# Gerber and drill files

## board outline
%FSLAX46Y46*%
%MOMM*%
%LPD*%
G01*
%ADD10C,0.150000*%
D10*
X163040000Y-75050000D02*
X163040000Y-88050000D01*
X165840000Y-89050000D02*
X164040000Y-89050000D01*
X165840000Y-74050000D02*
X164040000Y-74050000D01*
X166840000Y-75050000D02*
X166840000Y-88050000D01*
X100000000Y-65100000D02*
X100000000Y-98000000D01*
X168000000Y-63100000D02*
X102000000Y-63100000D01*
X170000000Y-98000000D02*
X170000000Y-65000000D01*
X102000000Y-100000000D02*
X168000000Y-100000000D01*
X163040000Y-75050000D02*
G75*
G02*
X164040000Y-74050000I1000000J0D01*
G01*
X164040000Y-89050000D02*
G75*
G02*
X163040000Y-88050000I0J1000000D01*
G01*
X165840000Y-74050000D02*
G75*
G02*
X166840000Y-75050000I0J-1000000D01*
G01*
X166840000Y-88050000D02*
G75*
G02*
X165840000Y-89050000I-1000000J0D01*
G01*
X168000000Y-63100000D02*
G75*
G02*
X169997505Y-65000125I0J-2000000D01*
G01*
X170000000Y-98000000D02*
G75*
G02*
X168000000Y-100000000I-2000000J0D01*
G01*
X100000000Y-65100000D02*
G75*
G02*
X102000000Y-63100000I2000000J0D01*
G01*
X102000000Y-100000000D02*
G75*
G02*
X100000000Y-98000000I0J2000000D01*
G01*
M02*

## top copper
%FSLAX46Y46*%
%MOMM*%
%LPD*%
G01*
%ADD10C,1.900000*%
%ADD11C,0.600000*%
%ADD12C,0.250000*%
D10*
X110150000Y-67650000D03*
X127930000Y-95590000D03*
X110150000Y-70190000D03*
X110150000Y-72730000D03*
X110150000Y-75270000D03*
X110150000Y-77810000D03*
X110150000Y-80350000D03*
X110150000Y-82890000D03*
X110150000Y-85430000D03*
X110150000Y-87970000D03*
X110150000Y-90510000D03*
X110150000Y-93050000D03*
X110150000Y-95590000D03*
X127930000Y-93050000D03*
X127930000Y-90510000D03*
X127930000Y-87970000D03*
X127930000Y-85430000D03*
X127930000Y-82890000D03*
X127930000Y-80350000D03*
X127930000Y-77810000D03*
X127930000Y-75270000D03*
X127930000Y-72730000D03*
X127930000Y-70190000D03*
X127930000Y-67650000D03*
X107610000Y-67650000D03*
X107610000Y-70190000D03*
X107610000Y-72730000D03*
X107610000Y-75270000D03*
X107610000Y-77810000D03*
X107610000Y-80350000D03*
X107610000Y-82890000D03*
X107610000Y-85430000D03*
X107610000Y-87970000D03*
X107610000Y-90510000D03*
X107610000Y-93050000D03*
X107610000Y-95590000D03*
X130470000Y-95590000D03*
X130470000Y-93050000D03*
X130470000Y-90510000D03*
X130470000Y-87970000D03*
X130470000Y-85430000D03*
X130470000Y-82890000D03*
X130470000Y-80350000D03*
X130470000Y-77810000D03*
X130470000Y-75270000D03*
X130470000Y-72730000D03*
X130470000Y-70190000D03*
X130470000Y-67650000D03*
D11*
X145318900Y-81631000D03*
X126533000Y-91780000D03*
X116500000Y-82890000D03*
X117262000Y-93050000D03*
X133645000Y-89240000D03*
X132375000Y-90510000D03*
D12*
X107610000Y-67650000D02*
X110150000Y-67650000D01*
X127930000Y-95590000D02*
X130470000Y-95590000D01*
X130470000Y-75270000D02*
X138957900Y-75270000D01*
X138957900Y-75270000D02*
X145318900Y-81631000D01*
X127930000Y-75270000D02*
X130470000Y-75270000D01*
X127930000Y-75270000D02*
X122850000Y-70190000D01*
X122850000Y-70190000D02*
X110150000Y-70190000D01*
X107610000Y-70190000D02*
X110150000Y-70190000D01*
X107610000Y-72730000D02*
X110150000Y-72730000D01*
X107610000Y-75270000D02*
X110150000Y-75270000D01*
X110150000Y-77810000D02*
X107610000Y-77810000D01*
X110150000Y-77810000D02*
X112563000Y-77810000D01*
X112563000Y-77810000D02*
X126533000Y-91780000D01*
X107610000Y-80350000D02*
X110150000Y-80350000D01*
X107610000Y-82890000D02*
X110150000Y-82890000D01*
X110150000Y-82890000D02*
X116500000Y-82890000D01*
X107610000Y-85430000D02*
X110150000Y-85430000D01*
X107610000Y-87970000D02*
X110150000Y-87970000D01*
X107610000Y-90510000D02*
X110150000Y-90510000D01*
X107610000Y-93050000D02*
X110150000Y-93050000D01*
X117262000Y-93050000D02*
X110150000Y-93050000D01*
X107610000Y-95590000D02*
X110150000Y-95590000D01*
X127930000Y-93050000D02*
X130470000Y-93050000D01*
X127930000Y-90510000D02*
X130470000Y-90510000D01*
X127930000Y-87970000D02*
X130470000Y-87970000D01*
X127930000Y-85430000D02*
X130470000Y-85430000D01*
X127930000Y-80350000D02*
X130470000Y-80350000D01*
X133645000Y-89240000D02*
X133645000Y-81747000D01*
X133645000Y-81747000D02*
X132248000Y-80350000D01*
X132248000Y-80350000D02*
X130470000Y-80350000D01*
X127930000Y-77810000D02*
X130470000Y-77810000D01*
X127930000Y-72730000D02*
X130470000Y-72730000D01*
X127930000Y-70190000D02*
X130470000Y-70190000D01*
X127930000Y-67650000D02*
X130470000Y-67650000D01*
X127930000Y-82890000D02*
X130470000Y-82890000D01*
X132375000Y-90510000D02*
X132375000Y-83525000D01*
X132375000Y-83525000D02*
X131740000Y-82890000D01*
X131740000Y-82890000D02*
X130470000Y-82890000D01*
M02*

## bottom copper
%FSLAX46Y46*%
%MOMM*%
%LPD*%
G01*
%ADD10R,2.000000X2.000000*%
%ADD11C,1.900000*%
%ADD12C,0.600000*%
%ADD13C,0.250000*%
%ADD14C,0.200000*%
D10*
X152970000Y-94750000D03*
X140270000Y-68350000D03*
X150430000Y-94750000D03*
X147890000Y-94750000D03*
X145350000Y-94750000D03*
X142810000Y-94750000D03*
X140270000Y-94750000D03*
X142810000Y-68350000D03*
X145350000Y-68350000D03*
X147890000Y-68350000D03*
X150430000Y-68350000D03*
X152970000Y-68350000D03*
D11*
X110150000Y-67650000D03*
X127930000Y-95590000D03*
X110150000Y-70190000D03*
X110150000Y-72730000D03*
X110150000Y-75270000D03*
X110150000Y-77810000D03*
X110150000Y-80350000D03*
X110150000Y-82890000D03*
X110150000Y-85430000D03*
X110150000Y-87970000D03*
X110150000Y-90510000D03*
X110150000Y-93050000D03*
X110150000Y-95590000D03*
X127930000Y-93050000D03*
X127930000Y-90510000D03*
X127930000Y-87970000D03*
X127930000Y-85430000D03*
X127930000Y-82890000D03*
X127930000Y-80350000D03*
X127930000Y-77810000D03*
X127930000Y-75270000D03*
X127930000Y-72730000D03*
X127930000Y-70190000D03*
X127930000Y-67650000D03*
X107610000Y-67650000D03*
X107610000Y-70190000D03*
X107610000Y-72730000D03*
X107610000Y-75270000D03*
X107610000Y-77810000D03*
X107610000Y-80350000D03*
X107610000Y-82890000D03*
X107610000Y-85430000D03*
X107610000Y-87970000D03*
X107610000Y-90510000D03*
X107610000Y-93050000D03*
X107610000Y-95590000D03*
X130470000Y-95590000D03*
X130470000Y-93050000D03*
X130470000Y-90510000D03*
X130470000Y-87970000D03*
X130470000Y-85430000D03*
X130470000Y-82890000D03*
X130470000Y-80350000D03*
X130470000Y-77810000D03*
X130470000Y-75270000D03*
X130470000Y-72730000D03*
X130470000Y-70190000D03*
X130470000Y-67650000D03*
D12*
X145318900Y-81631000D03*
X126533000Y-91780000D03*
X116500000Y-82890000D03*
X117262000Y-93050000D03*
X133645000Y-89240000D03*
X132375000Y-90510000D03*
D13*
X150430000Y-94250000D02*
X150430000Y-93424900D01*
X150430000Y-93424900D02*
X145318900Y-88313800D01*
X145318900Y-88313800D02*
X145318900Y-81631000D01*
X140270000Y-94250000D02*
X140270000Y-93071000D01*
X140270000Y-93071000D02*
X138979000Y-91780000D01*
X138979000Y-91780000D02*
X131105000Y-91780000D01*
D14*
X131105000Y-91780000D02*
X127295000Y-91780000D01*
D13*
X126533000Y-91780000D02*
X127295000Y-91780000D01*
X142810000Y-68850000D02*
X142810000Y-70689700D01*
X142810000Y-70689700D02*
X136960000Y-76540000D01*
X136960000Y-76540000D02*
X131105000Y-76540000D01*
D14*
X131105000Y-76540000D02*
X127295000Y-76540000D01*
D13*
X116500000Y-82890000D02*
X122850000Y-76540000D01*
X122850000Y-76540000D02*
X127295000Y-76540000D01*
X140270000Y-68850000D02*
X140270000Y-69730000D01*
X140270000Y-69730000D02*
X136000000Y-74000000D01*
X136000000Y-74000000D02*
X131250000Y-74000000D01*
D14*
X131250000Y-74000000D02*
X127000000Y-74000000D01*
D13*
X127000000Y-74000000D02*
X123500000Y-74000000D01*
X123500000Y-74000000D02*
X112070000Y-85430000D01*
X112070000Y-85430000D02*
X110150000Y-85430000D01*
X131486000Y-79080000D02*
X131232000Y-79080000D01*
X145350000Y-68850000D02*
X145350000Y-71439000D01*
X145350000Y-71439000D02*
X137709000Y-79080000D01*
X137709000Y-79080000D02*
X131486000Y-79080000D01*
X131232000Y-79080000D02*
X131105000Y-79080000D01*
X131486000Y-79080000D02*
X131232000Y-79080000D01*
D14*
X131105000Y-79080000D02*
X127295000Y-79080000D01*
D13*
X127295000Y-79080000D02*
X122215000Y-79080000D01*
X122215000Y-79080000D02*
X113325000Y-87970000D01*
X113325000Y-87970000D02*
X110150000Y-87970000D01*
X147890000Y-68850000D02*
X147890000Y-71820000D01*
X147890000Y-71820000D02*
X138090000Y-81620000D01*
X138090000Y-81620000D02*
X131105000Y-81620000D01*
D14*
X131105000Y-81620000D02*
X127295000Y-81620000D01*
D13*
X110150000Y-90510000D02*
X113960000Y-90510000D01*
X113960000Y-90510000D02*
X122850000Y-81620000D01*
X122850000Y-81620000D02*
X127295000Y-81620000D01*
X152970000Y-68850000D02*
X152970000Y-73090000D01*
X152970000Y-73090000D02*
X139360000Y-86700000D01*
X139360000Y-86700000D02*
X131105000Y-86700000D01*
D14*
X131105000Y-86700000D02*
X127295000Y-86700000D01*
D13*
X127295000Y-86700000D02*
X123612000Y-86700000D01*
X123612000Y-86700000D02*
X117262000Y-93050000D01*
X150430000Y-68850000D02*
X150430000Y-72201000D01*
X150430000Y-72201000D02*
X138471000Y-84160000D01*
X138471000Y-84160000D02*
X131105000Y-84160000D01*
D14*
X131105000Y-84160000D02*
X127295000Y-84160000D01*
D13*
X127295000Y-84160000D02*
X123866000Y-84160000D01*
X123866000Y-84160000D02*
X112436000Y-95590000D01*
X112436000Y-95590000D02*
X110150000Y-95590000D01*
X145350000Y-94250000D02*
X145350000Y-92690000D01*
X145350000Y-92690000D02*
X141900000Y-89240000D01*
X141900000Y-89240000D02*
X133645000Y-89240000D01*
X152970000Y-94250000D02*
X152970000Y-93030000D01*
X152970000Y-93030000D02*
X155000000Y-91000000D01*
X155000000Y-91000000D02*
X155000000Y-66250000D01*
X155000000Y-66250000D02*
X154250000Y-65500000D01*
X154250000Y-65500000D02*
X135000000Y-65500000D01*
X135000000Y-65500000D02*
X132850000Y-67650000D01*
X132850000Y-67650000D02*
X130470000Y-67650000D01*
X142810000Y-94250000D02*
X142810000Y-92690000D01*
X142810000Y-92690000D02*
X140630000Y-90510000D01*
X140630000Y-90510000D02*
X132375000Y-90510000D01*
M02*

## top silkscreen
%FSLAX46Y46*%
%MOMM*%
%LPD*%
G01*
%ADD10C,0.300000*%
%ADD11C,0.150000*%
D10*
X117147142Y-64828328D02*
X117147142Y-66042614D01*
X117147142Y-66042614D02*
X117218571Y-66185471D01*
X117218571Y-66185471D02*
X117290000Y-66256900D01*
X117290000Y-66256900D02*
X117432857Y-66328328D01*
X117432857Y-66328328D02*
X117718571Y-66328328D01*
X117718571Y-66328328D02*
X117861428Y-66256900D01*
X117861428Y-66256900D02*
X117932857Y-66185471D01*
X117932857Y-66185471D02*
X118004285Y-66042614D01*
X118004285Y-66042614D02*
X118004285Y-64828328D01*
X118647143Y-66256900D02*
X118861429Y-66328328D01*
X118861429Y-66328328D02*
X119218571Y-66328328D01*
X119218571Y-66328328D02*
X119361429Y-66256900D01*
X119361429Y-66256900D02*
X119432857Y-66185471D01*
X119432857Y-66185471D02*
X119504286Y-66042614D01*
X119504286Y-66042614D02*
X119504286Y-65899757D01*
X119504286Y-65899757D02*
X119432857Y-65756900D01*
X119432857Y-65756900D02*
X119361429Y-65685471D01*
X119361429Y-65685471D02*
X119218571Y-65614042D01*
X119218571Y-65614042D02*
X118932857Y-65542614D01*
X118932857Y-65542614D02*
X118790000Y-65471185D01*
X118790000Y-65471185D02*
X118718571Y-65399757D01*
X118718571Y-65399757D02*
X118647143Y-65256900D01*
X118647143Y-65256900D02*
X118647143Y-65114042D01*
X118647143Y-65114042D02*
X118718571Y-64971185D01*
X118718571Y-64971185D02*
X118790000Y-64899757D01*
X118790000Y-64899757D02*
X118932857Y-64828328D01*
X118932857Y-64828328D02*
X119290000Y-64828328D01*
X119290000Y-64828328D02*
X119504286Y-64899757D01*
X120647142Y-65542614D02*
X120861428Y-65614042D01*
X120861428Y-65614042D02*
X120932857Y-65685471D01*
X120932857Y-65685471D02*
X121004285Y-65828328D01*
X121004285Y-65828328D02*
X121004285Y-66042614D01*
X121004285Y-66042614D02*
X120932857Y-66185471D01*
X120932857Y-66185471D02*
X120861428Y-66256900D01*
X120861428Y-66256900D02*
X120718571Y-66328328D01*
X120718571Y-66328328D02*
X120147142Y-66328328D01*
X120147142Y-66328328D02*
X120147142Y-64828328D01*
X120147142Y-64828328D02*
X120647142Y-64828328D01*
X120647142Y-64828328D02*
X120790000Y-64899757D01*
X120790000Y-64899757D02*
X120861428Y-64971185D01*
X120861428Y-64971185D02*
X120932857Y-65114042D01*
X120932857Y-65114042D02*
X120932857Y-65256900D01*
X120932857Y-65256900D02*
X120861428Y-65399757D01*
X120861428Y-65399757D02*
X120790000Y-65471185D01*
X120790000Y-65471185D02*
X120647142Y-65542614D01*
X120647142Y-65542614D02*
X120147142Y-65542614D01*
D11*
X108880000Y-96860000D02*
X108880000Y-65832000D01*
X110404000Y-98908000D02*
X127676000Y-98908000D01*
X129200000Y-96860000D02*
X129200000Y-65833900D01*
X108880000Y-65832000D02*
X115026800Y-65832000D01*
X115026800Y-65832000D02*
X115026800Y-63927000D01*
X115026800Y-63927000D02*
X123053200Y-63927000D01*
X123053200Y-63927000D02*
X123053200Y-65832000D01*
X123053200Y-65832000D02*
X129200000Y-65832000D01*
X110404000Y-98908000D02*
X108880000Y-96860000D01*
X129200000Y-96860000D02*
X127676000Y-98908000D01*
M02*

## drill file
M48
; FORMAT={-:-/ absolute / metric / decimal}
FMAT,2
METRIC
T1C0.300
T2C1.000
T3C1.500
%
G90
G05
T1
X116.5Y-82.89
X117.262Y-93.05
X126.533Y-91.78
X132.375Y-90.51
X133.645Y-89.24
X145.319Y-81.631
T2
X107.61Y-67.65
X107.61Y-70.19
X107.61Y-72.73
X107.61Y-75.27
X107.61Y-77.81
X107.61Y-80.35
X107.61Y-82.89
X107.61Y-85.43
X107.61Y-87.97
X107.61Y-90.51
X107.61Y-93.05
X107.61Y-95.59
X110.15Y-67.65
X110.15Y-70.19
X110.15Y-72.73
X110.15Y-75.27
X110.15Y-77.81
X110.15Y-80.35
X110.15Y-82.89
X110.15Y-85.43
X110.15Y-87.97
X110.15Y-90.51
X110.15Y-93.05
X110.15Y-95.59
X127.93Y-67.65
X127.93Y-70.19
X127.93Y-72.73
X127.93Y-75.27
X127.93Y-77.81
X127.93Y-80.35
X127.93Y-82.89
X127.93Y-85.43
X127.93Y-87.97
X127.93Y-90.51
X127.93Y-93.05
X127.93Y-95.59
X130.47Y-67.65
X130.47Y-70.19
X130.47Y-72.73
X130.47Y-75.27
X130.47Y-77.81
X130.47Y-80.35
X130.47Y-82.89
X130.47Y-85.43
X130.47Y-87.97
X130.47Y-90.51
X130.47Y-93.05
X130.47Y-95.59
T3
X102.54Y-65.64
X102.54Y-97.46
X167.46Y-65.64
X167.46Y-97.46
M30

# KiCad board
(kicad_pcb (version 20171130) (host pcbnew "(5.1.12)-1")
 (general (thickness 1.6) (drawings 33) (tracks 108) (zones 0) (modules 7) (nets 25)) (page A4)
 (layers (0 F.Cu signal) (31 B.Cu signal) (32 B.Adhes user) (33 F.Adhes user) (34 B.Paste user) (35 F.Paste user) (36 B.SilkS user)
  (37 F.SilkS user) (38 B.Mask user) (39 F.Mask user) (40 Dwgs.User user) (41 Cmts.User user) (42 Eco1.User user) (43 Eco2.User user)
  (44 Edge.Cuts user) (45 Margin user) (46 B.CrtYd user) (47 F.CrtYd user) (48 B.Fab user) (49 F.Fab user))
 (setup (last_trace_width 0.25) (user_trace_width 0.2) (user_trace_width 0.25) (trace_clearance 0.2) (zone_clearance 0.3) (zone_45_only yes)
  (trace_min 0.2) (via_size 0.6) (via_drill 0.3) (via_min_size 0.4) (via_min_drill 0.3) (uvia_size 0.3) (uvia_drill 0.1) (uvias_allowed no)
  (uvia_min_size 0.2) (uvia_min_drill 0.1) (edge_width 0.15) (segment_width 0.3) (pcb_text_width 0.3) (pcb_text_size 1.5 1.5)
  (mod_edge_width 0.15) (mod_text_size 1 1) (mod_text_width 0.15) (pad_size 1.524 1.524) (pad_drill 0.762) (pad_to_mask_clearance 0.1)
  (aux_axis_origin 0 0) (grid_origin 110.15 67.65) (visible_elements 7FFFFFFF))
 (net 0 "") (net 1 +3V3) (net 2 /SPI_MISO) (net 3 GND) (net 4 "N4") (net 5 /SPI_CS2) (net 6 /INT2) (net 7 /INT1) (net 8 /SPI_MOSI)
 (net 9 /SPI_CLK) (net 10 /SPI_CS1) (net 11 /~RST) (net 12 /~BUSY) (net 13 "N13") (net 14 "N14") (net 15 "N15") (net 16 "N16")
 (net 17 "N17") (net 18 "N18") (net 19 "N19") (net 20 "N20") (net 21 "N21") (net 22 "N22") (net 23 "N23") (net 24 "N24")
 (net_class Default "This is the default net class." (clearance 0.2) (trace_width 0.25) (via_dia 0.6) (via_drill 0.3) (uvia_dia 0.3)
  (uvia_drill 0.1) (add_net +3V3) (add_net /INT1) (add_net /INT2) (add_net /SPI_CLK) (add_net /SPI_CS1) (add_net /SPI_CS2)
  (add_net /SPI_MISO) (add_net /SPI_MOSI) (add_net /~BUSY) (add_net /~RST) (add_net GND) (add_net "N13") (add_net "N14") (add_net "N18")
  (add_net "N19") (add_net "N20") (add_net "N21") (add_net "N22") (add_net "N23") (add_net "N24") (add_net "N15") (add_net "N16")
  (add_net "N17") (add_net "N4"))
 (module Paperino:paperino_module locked (layer B.Cu) (at 149.57 81.55 90)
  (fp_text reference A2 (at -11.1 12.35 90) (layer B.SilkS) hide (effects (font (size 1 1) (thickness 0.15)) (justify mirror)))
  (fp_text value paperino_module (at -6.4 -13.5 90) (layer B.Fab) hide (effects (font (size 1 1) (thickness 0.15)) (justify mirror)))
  (pad 1 smd rect (at -12.7 3.4 90) (size 2 2) (drill (offset -0.5 0)) (layers B.Cu B.Paste B.Mask) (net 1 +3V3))
  (pad 7 smd rect (at 12.7 -9.3 90) (size 2 2) (drill (offset 0.5 0)) (layers B.Cu B.Paste B.Mask) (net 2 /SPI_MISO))
  (pad 2 smd rect (at -12.7 0.86 90) (size 2 2) (drill (offset -0.5 0)) (layers B.Cu B.Paste B.Mask) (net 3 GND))
  (pad 3 smd rect (at -12.7 -1.68 90) (size 2 2) (drill (offset -0.5 0)) (layers B.Cu B.Paste B.Mask) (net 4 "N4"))
  (pad 4 smd rect (at -12.7 -4.22 90) (size 2 2) (drill (offset -0.5 0)) (layers B.Cu B.Paste B.Mask) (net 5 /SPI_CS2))
  (pad 5 smd rect (at -12.7 -6.76 90) (size 2 2) (drill (offset -0.5 0)) (layers B.Cu B.Paste B.Mask) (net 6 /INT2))
  (pad 6 smd rect (at -12.7 -9.3 90) (size 2 2) (drill (offset -0.5 0)) (layers B.Cu B.Paste B.Mask) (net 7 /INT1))
  (pad 8 smd rect (at 12.7 -6.76 90) (size 2 2) (drill (offset 0.5 0)) (layers B.Cu B.Paste B.Mask) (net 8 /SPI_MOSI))
  (pad 9 smd rect (at 12.7 -4.22 90) (size 2 2) (drill (offset 0.5 0)) (layers B.Cu B.Paste B.Mask) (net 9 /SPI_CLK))
  (pad 10 smd rect (at 12.7 -1.68 90) (size 2 2) (drill (offset 0.5 0)) (layers B.Cu B.Paste B.Mask) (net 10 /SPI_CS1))
  (pad 11 smd rect (at 12.7 0.86 90) (size 2 2) (drill (offset 0.5 0)) (layers B.Cu B.Paste B.Mask) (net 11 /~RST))
  (pad 12 smd rect (at 12.7 3.4 90) (size 2 2) (drill (offset 0.5 0)) (layers B.Cu B.Paste B.Mask) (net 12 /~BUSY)))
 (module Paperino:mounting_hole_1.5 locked (layer F.Cu) (at 102.54 97.46)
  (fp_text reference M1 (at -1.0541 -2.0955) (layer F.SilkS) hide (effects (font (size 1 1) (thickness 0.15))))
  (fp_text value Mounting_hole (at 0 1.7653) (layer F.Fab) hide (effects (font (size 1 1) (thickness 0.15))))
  (pad "" np_thru_hole circle (at 0 0) (size 1.5 1.5) (drill 1.5) (layers *.Cu *.Mask)))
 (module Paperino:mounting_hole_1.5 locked (layer F.Cu) (at 167.46 65.64)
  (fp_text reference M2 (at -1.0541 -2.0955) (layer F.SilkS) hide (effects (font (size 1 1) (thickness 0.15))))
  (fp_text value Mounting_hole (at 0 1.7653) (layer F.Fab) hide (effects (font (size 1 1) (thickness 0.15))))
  (pad "" np_thru_hole circle (at 0 0) (size 1.5 1.5) (drill 1.5) (layers *.Cu *.Mask)))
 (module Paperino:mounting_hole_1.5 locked (layer F.Cu) (at 102.54 65.64)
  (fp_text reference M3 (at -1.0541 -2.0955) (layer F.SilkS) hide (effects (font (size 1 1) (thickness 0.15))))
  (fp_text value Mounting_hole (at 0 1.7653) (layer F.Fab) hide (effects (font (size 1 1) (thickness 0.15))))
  (pad "" np_thru_hole circle (at 0 0) (size 1.5 1.5) (drill 1.5) (layers *.Cu *.Mask)))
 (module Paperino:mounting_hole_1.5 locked (layer F.Cu) (at 167.46 97.46)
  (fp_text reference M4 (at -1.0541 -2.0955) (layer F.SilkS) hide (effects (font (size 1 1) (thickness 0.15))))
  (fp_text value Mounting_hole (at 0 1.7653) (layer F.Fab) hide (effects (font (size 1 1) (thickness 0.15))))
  (pad "" np_thru_hole circle (at 0 0) (size 1.5 1.5) (drill 1.5) (layers *.Cu *.Mask)))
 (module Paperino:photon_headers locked (layer F.Cu) (at 108.88 99.908)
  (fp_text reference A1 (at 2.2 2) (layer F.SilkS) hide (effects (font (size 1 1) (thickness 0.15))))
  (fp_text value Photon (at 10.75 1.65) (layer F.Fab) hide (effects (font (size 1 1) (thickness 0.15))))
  (fp_line (start 0 -3.048) (end 0 -34.076) (layer F.SilkS) (width 0.15))
  (fp_line (start 1.524 -1) (end 18.796 -1) (layer F.SilkS) (width 0.15))
  (fp_line (start 20.32 -3.048) (end 20.32 -34.0741) (layer F.SilkS) (width 0.15))
  (fp_line (start 0 -34.076) (end 6.1468 -34.076) (layer F.SilkS) (width 0.15))
  (fp_line (start 6.1468 -34.076) (end 6.1468 -35.981) (layer F.SilkS) (width 0.15))
  (fp_line (start 6.1468 -35.981) (end 14.1732 -35.981) (layer F.SilkS) (width 0.15))
  (fp_line (start 14.1732 -35.981) (end 14.1732 -34.076) (layer F.SilkS) (width 0.15))
  (fp_line (start 14.1732 -34.076) (end 20.32 -34.076) (layer F.SilkS) (width 0.15))
  (fp_line (start 1.524 -1) (end 0 -3.048) (layer F.SilkS) (width 0.15))
  (fp_line (start 20.32 -3.048) (end 18.796 -1) (layer F.SilkS) (width 0.15))
  (pad 1 thru_hole circle (at 1.27 -32.258) (size 1.9 1.9) (drill 1) (layers *.Cu *.Mask) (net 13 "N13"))
  (pad 13 thru_hole circle (at 19.05 -4.318) (size 1.9 1.9) (drill 1) (layers *.Cu *.Mask) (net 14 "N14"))
  (pad 2 thru_hole circle (at 1.27 -29.718) (size 1.9 1.9) (drill 1) (layers *.Cu *.Mask) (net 3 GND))
  (pad 3 thru_hole circle (at 1.27 -27.178) (size 1.9 1.9) (drill 1) (layers *.Cu *.Mask) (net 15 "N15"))
  (pad 4 thru_hole circle (at 1.27 -24.638) (size 1.9 1.9) (drill 1) (layers *.Cu *.Mask) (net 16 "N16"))
  (pad 5 thru_hole circle (at 1.27 -22.098) (size 1.9 1.9) (drill 1) (layers *.Cu *.Mask) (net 7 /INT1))
  (pad 6 thru_hole circle (at 1.27 -19.558) (size 1.9 1.9) (drill 1) (layers *.Cu *.Mask) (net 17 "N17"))
  (pad 7 thru_hole circle (at 1.27 -17.018) (size 1.9 1.9) (drill 1) (layers *.Cu *.Mask) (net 8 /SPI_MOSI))
  (pad 8 thru_hole circle (at 1.27 -14.478) (size 1.9 1.9) (drill 1) (layers *.Cu *.Mask) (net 2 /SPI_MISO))
  (pad 9 thru_hole circle (at 1.27 -11.938) (size 1.9 1.9) (drill 1) (layers *.Cu *.Mask) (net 9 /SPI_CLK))
  (pad 10 thru_hole circle (at 1.27 -9.398) (size 1.9 1.9) (drill 1) (layers *.Cu *.Mask) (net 10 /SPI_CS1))
  (pad 11 thru_hole circle (at 1.27 -6.858) (size 1.9 1.9) (drill 1) (layers *.Cu *.Mask) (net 12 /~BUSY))
  (pad 12 thru_hole circle (at 1.27 -4.318) (size 1.9 1.9) (drill 1) (layers *.Cu *.Mask) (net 11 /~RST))
  (pad 14 thru_hole circle (at 19.05 -6.858) (size 1.9 1.9) (drill 1) (layers *.Cu *.Mask) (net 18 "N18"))
  (pad 15 thru_hole circle (at 19.05 -9.398) (size 1.9 1.9) (drill 1) (layers *.Cu *.Mask) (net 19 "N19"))
  (pad 16 thru_hole circle (at 19.05 -11.938) (size 1.9 1.9) (drill 1) (layers *.Cu *.Mask) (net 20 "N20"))
  (pad 17 thru_hole circle (at 19.05 -14.478) (size 1.9 1.9) (drill 1) (layers *.Cu *.Mask) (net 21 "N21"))
  (pad 18 thru_hole circle (at 19.05 -17.018) (size 1.9 1.9) (drill 1) (layers *.Cu *.Mask) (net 6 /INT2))
  (pad 19 thru_hole circle (at 19.05 -19.558) (size 1.9 1.9) (drill 1) (layers *.Cu *.Mask) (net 5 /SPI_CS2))
  (pad 20 thru_hole circle (at 19.05 -22.098) (size 1.9 1.9) (drill 1) (layers *.Cu *.Mask) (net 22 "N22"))
  (pad 21 thru_hole circle (at 19.05 -24.638) (size 1.9 1.9) (drill 1) (layers *.Cu *.Mask) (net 3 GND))
  (pad 22 thru_hole circle (at 19.05 -27.178) (size 1.9 1.9) (drill 1) (layers *.Cu *.Mask) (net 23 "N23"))
  (pad 23 thru_hole circle (at 19.05 -29.718) (size 1.9 1.9) (drill 1) (layers *.Cu *.Mask) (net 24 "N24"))
  (pad 24 thru_hole circle (at 19.05 -32.258) (size 1.9 1.9) (drill 1) (layers *.Cu *.Mask) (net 1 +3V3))
  (pad 1 thru_hole circle (at -1.27 -32.258) (size 1.9 1.9) (drill 1) (layers *.Cu *.Mask) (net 13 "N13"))
  (pad 2 thru_hole circle (at -1.27 -29.718) (size 1.9 1.9) (drill 1) (layers *.Cu *.Mask) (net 3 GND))
  (pad 3 thru_hole circle (at -1.27 -27.178) (size 1.9 1.9) (drill 1) (layers *.Cu *.Mask) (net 15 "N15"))
  (pad 4 thru_hole circle (at -1.27 -24.638) (size 1.9 1.9) (drill 1) (layers *.Cu *.Mask) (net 16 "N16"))
  (pad 5 thru_hole circle (at -1.27 -22.098) (size 1.9 1.9) (drill 1) (layers *.Cu *.Mask) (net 7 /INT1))
  (pad 6 thru_hole circle (at -1.27 -19.558) (size 1.9 1.9) (drill 1) (layers *.Cu *.Mask) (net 17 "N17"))
  (pad 7 thru_hole circle (at -1.27 -17.018) (size 1.9 1.9) (drill 1) (layers *.Cu *.Mask) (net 8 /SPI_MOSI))
  (pad 8 thru_hole circle (at -1.27 -14.478) (size 1.9 1.9) (drill 1) (layers *.Cu *.Mask) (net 2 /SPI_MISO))
  (pad 9 thru_hole circle (at -1.27 -11.938) (size 1.9 1.9) (drill 1) (layers *.Cu *.Mask) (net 9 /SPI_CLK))
  (pad 10 thru_hole circle (at -1.27 -9.398) (size 1.9 1.9) (drill 1) (layers *.Cu *.Mask) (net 10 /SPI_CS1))
  (pad 11 thru_hole circle (at -1.27 -6.858) (size 1.9 1.9) (drill 1) (layers *.Cu *.Mask) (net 12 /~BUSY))
  (pad 12 thru_hole circle (at -1.27 -4.318) (size 1.9 1.9) (drill 1) (layers *.Cu *.Mask) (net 11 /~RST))
  (pad 13 thru_hole circle (at 21.59 -4.318) (size 1.9 1.9) (drill 1) (layers *.Cu *.Mask) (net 14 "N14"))
  (pad 14 thru_hole circle (at 21.59 -6.858) (size 1.9 1.9) (drill 1) (layers *.Cu *.Mask) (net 18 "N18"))
  (pad 15 thru_hole circle (at 21.59 -9.398) (size 1.9 1.9) (drill 1) (layers *.Cu *.Mask) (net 19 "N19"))
  (pad 16 thru_hole circle (at 21.59 -11.938) (size 1.9 1.9) (drill 1) (layers *.Cu *.Mask) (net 20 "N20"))
  (pad 17 thru_hole circle (at 21.59 -14.478) (size 1.9 1.9) (drill 1) (layers *.Cu *.Mask) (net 21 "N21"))
  (pad 18 thru_hole circle (at 21.59 -17.018) (size 1.9 1.9) (drill 1) (layers *.Cu *.Mask) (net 6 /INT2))
  (pad 19 thru_hole circle (at 21.59 -19.558) (size 1.9 1.9) (drill 1) (layers *.Cu *.Mask) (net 5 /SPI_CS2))
  (pad 20 thru_hole circle (at 21.59 -22.098) (size 1.9 1.9) (drill 1) (layers *.Cu *.Mask) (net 22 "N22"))
  (pad 21 thru_hole circle (at 21.59 -24.638) (size 1.9 1.9) (drill 1) (layers *.Cu *.Mask) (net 3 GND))
  (pad 22 thru_hole circle (at 21.59 -27.178) (size 1.9 1.9) (drill 1) (layers *.Cu *.Mask) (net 23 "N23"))
  (pad 23 thru_hole circle (at 21.59 -29.718) (size 1.9 1.9) (drill 1) (layers *.Cu *.Mask) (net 24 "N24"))
  (pad 24 thru_hole circle (at 21.59 -32.258) (size 1.9 1.9) (drill 1) (layers *.Cu *.Mask) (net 1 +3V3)))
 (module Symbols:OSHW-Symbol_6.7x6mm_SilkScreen (layer B.Cu) (at 118.786 93.05 270)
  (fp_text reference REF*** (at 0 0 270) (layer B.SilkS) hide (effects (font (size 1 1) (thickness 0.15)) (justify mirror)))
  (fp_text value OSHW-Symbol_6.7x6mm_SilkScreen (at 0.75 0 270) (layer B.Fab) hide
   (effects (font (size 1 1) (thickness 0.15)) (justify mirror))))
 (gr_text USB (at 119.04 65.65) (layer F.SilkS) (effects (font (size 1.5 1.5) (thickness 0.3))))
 (gr_line (start 163.04 75.05) (end 163.04 88.05) (layer Edge.Cuts) (width 0.15))
 (gr_line (start 165.84 89.05) (end 164.04 89.05) (layer Edge.Cuts) (width 0.15))
 (gr_line (start 165.84 74.05) (end 164.04 74.05) (layer Edge.Cuts) (width 0.15))
 (gr_line (start 166.84 75.05) (end 166.84 88.05) (layer Edge.Cuts) (width 0.15))
 (gr_line (start 100 65.1) (end 100 98) (layer Edge.Cuts) (width 0.15))
 (gr_line (start 168 63.1) (end 102 63.1) (layer Edge.Cuts) (width 0.15))
 (gr_line (start 170 98) (end 170 65) (layer Edge.Cuts) (width 0.15))
 (gr_line (start 102 100) (end 168 100) (layer Edge.Cuts) (width 0.15))
 (gr_arc (start 164.04 75.05) (end 164.04 74.05) (angle -90) (layer Edge.Cuts) (width 0.15))
 (gr_arc (start 164.04 88.05) (end 164.04 89.05) (angle 90) (layer Edge.Cuts) (width 0.15))
 (gr_arc (start 165.84 75.05) (end 165.84 74.05) (angle 90) (layer Edge.Cuts) (width 0.15))
 (gr_arc (start 165.84 88.05) (end 166.84 88.05) (angle 90) (layer Edge.Cuts) (width 0.15))
 (gr_arc (start 168 65.1) (end 168 63.1) (angle 87.13759477) (layer Edge.Cuts) (width 0.15))
 (gr_arc (start 168 98) (end 170 98) (angle 90) (layer Edge.Cuts) (width 0.15))
 (gr_arc (start 102 65.1) (end 100 65.1) (angle 90) (layer Edge.Cuts) (width 0.15))
 (gr_arc (start 102 98) (end 102 100) (angle 90) (layer Edge.Cuts) (width 0.15))
 (segment (start 107.61 67.65) (end 110.15 67.65) (width 0.25) (layer F.Cu) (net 13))
 (segment (start 127.93 95.59) (end 130.47 95.59) (width 0.25) (layer F.Cu) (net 14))
 (segment (start 150.43 94.25) (end 150.43 93.4249) (width 0.25) (layer B.Cu) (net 3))
 (segment (start 130.47 75.27) (end 138.9579 75.27) (width 0.25) (layer F.Cu) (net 3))
 (segment (start 138.9579 75.27) (end 145.3189 81.631) (width 0.25) (layer F.Cu) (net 3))
 (segment (start 150.43 93.4249) (end 145.3189 88.3138) (width 0.25) (layer B.Cu) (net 3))
 (segment (start 145.3189 88.3138) (end 145.3189 81.631) (width 0.25) (layer B.Cu) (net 3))
 (segment (start 127.93 75.27) (end 130.47 75.27) (width 0.25) (layer F.Cu) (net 3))
 (segment (start 127.93 75.27) (end 122.85 70.19) (width 0.25) (layer F.Cu) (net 3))
 (segment (start 122.85 70.19) (end 110.15 70.19) (width 0.25) (layer F.Cu) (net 3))
 (segment (start 107.61 70.19) (end 110.15 70.19) (width 0.25) (layer F.Cu) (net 3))
 (via (at 145.3189 81.631) (size 0.6) (layers F.Cu B.Cu) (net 3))
 (segment (start 107.61 72.73) (end 110.15 72.73) (width 0.25) (layer F.Cu) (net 15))
 (segment (start 107.61 75.27) (end 110.15 75.27) (width 0.25) (layer F.Cu) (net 16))
 (segment (start 110.15 77.81) (end 107.61 77.81) (width 0.25) (layer F.Cu) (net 7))
 (segment (start 140.27 94.25) (end 140.27 93.071) (width 0.25) (layer B.Cu) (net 7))
 (segment (start 140.27 93.071) (end 138.979 91.78) (width 0.25) (layer B.Cu) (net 7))
 (segment (start 138.979 91.78) (end 131.105 91.78) (width 0.25) (layer B.Cu) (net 7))
 (segment (start 131.105 91.78) (end 127.295 91.78) (width 0.2) (layer B.Cu) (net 7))
 (segment (start 110.15 77.81) (end 112.563 77.81) (width 0.25) (layer F.Cu) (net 7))
 (segment (start 112.563 77.81) (end 126.533 91.78) (width 0.25) (layer F.Cu) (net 7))
 (segment (start 126.533 91.78) (end 127.295 91.78) (width 0.25) (layer B.Cu) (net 7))
 (via (at 126.533 91.78) (size 0.6) (layers F.Cu B.Cu) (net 7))
 (segment (start 107.61 80.35) (end 110.15 80.35) (width 0.25) (layer F.Cu) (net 17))
 (segment (start 107.61 82.89) (end 110.15 82.89) (width 0.25) (layer F.Cu) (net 8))
 (segment (start 142.81 68.85) (end 142.81 70.6897) (width 0.25) (layer B.Cu) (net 8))
 (segment (start 142.81 70.6897) (end 136.96 76.54) (width 0.25) (layer B.Cu) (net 8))
 (segment (start 136.96 76.54) (end 131.105 76.54) (width 0.25) (layer B.Cu) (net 8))
 (segment (start 131.105 76.54) (end 127.295 76.54) (width 0.2) (layer B.Cu) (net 8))
 (segment (start 110.15 82.89) (end 116.5 82.89) (width 0.25) (layer F.Cu) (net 8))
 (segment (start 116.5 82.89) (end 122.85 76.54) (width 0.25) (layer B.Cu) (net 8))
 (segment (start 122.85 76.54) (end 127.295 76.54) (width 0.25) (layer B.Cu) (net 8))
 (via (at 116.5 82.89) (size 0.6) (layers F.Cu B.Cu) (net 8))
 (segment (start 107.61 85.43) (end 110.15 85.43) (width 0.25) (layer F.Cu) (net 2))
 (segment (start 140.27 68.85) (end 140.27 69.73) (width 0.25) (layer B.Cu) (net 2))
 (segment (start 140.27 69.73) (end 136 74) (width 0.25) (layer B.Cu) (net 2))
 (segment (start 136 74) (end 131.25 74) (width 0.25) (layer B.Cu) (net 2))
 (segment (start 131.25 74) (end 127 74) (width 0.2) (layer B.Cu) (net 2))
 (segment (start 127 74) (end 123.5 74) (width 0.25) (layer B.Cu) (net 2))
 (segment (start 123.5 74) (end 112.07 85.43) (width 0.25) (layer B.Cu) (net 2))
 (segment (start 112.07 85.43) (end 110.15 85.43) (width 0.25) (layer B.Cu) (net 2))
 (segment (start 131.486 79.08) (end 131.232 79.08) (width 0.25) (layer B.Cu) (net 9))
 (segment (start 145.35 68.85) (end 145.35 71.439) (width 0.25) (layer B.Cu) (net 9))
 (segment (start 145.35 71.439) (end 137.709 79.08) (width 0.25) (layer B.Cu) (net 9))
 (segment (start 137.709 79.08) (end 131.486 79.08) (width 0.25) (layer B.Cu) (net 9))
 (segment (start 131.232 79.08) (end 131.105 79.08) (width 0.25) (layer B.Cu) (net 9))
 (segment (start 107.61 87.97) (end 110.15 87.97) (width 0.25) (layer F.Cu) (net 9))
 (segment (start 131.486 79.08) (end 131.232 79.08) (width 0.25) (layer B.Cu) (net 9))
 (segment (start 131.105 79.08) (end 127.295 79.08) (width 0.2) (layer B.Cu) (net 9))
 (segment (start 127.295 79.08) (end 122.215 79.08) (width 0.25) (layer B.Cu) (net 9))
 (segment (start 122.215 79.08) (end 113.325 87.97) (width 0.25) (layer B.Cu) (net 9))
 (segment (start 113.325 87.97) (end 110.15 87.97) (width 0.25) (layer B.Cu) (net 9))
 (segment (start 107.61 90.51) (end 110.15 90.51) (width 0.25) (layer F.Cu) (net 10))
 (segment (start 147.89 68.85) (end 147.89 71.82) (width 0.25) (layer B.Cu) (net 10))
 (segment (start 147.89 71.82) (end 138.09 81.62) (width 0.25) (layer B.Cu) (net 10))
 (segment (start 138.09 81.62) (end 131.105 81.62) (width 0.25) (layer B.Cu) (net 10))
 (segment (start 131.105 81.62) (end 127.295 81.62) (width 0.2) (layer B.Cu) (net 10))
 (segment (start 110.15 90.51) (end 113.96 90.51) (width 0.25) (layer B.Cu) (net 10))
 (segment (start 113.96 90.51) (end 122.85 81.62) (width 0.25) (layer B.Cu) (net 10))
 (segment (start 122.85 81.62) (end 127.295 81.62) (width 0.25) (layer B.Cu) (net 10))
 (segment (start 107.61 93.05) (end 110.15 93.05) (width 0.25) (layer F.Cu) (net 12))
 (segment (start 152.97 68.85) (end 152.97 73.09) (width 0.25) (layer B.Cu) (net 12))
 (segment (start 152.97 73.09) (end 139.36 86.7) (width 0.25) (layer B.Cu) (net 12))
 (segment (start 139.36 86.7) (end 131.105 86.7) (width 0.25) (layer B.Cu) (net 12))
 (segment (start 131.105 86.7) (end 127.295 86.7) (width 0.2) (layer B.Cu) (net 12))
 (segment (start 127.295 86.7) (end 123.612 86.7) (width 0.25) (layer B.Cu) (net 12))
 (segment (start 123.612 86.7) (end 117.262 93.05) (width 0.25) (layer B.Cu) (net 12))
 (segment (start 117.262 93.05) (end 110.15 93.05) (width 0.25) (layer F.Cu) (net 12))
 (via (at 117.262 93.05) (size 0.6) (layers F.Cu B.Cu) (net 12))
 (segment (start 107.61 95.59) (end 110.15 95.59) (width 0.25) (layer F.Cu) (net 11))
 (segment (start 150.43 68.85) (end 150.43 72.201) (width 0.25) (layer B.Cu) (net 11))
 (segment (start 150.43 72.201) (end 138.471 84.16) (width 0.25) (layer B.Cu) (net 11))
 (segment (start 138.471 84.16) (end 131.105 84.16) (width 0.25) (layer B.Cu) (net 11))
 (segment (start 131.105 84.16) (end 127.295 84.16) (width 0.2) (layer B.Cu) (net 11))
 (segment (start 127.295 84.16) (end 123.866 84.16) (width 0.25) (layer B.Cu) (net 11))
 (segment (start 123.866 84.16) (end 112.436 95.59) (width 0.25) (layer B.Cu) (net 11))
 (segment (start 112.436 95.59) (end 110.15 95.59) (width 0.25) (layer B.Cu) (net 11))
 (segment (start 127.93 93.05) (end 130.47 93.05) (width 0.25) (layer F.Cu) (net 18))
 (segment (start 127.93 90.51) (end 130.47 90.51) (width 0.25) (layer F.Cu) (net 19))
 (segment (start 127.93 87.97) (end 130.47 87.97) (width 0.25) (layer F.Cu) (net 20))
 (segment (start 127.93 85.43) (end 130.47 85.43) (width 0.25) (layer F.Cu) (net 21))
 (segment (start 127.93 80.35) (end 130.47 80.35) (width 0.25) (layer F.Cu) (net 5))
 (segment (start 145.35 94.25) (end 145.35 92.69) (width 0.25) (layer B.Cu) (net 5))
 (segment (start 145.35 92.69) (end 141.9 89.24) (width 0.25) (layer B.Cu) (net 5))
 (segment (start 141.9 89.24) (end 133.645 89.24) (width 0.25) (layer B.Cu) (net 5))
 (segment (start 133.645 89.24) (end 133.645 81.747) (width 0.25) (layer F.Cu) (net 5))
 (segment (start 133.645 81.747) (end 132.248 80.35) (width 0.25) (layer F.Cu) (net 5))
 (segment (start 132.248 80.35) (end 130.47 80.35) (width 0.25) (layer F.Cu) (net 5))
 (via (at 133.645 89.24) (size 0.6) (layers F.Cu B.Cu) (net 5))
 (segment (start 127.93 77.81) (end 130.47 77.81) (width 0.25) (layer F.Cu) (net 22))
 (segment (start 127.93 72.73) (end 130.47 72.73) (width 0.25) (layer F.Cu) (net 23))
 (segment (start 127.93 70.19) (end 130.47 70.19) (width 0.25) (layer F.Cu) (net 24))
 (segment (start 127.93 67.65) (end 130.47 67.65) (width 0.25) (layer F.Cu) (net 1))
 (segment (start 152.97 94.25) (end 152.97 93.03) (width 0.25) (layer B.Cu) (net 1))
 (segment (start 152.97 93.03) (end 155 91) (width 0.25) (layer B.Cu) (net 1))
 (segment (start 155 91) (end 155 66.25) (width 0.25) (layer B.Cu) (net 1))
 (segment (start 155 66.25) (end 154.25 65.5) (width 0.25) (layer B.Cu) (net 1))
 (segment (start 154.25 65.5) (end 135 65.5) (width 0.25) (layer B.Cu) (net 1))
 (segment (start 135 65.5) (end 132.85 67.65) (width 0.25) (layer B.Cu) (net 1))
 (segment (start 132.85 67.65) (end 130.47 67.65) (width 0.25) (layer B.Cu) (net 1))
 (segment (start 127.93 82.89) (end 130.47 82.89) (width 0.25) (layer F.Cu) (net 6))
 (segment (start 142.81 94.25) (end 142.81 92.69) (width 0.25) (layer B.Cu) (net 6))
 (segment (start 142.81 92.69) (end 140.63 90.51) (width 0.25) (layer B.Cu) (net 6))
 (segment (start 140.63 90.51) (end 132.375 90.51) (width 0.25) (layer B.Cu) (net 6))
 (segment (start 132.375 90.51) (end 132.375 83.525) (width 0.25) (layer F.Cu) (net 6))
 (segment (start 132.375 83.525) (end 131.74 82.89) (width 0.25) (layer F.Cu) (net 6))
 (segment (start 131.74 82.89) (end 130.47 82.89) (width 0.25) (layer F.Cu) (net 6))
 (via (at 132.375 90.51) (size 0.6) (layers F.Cu B.Cu) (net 6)))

